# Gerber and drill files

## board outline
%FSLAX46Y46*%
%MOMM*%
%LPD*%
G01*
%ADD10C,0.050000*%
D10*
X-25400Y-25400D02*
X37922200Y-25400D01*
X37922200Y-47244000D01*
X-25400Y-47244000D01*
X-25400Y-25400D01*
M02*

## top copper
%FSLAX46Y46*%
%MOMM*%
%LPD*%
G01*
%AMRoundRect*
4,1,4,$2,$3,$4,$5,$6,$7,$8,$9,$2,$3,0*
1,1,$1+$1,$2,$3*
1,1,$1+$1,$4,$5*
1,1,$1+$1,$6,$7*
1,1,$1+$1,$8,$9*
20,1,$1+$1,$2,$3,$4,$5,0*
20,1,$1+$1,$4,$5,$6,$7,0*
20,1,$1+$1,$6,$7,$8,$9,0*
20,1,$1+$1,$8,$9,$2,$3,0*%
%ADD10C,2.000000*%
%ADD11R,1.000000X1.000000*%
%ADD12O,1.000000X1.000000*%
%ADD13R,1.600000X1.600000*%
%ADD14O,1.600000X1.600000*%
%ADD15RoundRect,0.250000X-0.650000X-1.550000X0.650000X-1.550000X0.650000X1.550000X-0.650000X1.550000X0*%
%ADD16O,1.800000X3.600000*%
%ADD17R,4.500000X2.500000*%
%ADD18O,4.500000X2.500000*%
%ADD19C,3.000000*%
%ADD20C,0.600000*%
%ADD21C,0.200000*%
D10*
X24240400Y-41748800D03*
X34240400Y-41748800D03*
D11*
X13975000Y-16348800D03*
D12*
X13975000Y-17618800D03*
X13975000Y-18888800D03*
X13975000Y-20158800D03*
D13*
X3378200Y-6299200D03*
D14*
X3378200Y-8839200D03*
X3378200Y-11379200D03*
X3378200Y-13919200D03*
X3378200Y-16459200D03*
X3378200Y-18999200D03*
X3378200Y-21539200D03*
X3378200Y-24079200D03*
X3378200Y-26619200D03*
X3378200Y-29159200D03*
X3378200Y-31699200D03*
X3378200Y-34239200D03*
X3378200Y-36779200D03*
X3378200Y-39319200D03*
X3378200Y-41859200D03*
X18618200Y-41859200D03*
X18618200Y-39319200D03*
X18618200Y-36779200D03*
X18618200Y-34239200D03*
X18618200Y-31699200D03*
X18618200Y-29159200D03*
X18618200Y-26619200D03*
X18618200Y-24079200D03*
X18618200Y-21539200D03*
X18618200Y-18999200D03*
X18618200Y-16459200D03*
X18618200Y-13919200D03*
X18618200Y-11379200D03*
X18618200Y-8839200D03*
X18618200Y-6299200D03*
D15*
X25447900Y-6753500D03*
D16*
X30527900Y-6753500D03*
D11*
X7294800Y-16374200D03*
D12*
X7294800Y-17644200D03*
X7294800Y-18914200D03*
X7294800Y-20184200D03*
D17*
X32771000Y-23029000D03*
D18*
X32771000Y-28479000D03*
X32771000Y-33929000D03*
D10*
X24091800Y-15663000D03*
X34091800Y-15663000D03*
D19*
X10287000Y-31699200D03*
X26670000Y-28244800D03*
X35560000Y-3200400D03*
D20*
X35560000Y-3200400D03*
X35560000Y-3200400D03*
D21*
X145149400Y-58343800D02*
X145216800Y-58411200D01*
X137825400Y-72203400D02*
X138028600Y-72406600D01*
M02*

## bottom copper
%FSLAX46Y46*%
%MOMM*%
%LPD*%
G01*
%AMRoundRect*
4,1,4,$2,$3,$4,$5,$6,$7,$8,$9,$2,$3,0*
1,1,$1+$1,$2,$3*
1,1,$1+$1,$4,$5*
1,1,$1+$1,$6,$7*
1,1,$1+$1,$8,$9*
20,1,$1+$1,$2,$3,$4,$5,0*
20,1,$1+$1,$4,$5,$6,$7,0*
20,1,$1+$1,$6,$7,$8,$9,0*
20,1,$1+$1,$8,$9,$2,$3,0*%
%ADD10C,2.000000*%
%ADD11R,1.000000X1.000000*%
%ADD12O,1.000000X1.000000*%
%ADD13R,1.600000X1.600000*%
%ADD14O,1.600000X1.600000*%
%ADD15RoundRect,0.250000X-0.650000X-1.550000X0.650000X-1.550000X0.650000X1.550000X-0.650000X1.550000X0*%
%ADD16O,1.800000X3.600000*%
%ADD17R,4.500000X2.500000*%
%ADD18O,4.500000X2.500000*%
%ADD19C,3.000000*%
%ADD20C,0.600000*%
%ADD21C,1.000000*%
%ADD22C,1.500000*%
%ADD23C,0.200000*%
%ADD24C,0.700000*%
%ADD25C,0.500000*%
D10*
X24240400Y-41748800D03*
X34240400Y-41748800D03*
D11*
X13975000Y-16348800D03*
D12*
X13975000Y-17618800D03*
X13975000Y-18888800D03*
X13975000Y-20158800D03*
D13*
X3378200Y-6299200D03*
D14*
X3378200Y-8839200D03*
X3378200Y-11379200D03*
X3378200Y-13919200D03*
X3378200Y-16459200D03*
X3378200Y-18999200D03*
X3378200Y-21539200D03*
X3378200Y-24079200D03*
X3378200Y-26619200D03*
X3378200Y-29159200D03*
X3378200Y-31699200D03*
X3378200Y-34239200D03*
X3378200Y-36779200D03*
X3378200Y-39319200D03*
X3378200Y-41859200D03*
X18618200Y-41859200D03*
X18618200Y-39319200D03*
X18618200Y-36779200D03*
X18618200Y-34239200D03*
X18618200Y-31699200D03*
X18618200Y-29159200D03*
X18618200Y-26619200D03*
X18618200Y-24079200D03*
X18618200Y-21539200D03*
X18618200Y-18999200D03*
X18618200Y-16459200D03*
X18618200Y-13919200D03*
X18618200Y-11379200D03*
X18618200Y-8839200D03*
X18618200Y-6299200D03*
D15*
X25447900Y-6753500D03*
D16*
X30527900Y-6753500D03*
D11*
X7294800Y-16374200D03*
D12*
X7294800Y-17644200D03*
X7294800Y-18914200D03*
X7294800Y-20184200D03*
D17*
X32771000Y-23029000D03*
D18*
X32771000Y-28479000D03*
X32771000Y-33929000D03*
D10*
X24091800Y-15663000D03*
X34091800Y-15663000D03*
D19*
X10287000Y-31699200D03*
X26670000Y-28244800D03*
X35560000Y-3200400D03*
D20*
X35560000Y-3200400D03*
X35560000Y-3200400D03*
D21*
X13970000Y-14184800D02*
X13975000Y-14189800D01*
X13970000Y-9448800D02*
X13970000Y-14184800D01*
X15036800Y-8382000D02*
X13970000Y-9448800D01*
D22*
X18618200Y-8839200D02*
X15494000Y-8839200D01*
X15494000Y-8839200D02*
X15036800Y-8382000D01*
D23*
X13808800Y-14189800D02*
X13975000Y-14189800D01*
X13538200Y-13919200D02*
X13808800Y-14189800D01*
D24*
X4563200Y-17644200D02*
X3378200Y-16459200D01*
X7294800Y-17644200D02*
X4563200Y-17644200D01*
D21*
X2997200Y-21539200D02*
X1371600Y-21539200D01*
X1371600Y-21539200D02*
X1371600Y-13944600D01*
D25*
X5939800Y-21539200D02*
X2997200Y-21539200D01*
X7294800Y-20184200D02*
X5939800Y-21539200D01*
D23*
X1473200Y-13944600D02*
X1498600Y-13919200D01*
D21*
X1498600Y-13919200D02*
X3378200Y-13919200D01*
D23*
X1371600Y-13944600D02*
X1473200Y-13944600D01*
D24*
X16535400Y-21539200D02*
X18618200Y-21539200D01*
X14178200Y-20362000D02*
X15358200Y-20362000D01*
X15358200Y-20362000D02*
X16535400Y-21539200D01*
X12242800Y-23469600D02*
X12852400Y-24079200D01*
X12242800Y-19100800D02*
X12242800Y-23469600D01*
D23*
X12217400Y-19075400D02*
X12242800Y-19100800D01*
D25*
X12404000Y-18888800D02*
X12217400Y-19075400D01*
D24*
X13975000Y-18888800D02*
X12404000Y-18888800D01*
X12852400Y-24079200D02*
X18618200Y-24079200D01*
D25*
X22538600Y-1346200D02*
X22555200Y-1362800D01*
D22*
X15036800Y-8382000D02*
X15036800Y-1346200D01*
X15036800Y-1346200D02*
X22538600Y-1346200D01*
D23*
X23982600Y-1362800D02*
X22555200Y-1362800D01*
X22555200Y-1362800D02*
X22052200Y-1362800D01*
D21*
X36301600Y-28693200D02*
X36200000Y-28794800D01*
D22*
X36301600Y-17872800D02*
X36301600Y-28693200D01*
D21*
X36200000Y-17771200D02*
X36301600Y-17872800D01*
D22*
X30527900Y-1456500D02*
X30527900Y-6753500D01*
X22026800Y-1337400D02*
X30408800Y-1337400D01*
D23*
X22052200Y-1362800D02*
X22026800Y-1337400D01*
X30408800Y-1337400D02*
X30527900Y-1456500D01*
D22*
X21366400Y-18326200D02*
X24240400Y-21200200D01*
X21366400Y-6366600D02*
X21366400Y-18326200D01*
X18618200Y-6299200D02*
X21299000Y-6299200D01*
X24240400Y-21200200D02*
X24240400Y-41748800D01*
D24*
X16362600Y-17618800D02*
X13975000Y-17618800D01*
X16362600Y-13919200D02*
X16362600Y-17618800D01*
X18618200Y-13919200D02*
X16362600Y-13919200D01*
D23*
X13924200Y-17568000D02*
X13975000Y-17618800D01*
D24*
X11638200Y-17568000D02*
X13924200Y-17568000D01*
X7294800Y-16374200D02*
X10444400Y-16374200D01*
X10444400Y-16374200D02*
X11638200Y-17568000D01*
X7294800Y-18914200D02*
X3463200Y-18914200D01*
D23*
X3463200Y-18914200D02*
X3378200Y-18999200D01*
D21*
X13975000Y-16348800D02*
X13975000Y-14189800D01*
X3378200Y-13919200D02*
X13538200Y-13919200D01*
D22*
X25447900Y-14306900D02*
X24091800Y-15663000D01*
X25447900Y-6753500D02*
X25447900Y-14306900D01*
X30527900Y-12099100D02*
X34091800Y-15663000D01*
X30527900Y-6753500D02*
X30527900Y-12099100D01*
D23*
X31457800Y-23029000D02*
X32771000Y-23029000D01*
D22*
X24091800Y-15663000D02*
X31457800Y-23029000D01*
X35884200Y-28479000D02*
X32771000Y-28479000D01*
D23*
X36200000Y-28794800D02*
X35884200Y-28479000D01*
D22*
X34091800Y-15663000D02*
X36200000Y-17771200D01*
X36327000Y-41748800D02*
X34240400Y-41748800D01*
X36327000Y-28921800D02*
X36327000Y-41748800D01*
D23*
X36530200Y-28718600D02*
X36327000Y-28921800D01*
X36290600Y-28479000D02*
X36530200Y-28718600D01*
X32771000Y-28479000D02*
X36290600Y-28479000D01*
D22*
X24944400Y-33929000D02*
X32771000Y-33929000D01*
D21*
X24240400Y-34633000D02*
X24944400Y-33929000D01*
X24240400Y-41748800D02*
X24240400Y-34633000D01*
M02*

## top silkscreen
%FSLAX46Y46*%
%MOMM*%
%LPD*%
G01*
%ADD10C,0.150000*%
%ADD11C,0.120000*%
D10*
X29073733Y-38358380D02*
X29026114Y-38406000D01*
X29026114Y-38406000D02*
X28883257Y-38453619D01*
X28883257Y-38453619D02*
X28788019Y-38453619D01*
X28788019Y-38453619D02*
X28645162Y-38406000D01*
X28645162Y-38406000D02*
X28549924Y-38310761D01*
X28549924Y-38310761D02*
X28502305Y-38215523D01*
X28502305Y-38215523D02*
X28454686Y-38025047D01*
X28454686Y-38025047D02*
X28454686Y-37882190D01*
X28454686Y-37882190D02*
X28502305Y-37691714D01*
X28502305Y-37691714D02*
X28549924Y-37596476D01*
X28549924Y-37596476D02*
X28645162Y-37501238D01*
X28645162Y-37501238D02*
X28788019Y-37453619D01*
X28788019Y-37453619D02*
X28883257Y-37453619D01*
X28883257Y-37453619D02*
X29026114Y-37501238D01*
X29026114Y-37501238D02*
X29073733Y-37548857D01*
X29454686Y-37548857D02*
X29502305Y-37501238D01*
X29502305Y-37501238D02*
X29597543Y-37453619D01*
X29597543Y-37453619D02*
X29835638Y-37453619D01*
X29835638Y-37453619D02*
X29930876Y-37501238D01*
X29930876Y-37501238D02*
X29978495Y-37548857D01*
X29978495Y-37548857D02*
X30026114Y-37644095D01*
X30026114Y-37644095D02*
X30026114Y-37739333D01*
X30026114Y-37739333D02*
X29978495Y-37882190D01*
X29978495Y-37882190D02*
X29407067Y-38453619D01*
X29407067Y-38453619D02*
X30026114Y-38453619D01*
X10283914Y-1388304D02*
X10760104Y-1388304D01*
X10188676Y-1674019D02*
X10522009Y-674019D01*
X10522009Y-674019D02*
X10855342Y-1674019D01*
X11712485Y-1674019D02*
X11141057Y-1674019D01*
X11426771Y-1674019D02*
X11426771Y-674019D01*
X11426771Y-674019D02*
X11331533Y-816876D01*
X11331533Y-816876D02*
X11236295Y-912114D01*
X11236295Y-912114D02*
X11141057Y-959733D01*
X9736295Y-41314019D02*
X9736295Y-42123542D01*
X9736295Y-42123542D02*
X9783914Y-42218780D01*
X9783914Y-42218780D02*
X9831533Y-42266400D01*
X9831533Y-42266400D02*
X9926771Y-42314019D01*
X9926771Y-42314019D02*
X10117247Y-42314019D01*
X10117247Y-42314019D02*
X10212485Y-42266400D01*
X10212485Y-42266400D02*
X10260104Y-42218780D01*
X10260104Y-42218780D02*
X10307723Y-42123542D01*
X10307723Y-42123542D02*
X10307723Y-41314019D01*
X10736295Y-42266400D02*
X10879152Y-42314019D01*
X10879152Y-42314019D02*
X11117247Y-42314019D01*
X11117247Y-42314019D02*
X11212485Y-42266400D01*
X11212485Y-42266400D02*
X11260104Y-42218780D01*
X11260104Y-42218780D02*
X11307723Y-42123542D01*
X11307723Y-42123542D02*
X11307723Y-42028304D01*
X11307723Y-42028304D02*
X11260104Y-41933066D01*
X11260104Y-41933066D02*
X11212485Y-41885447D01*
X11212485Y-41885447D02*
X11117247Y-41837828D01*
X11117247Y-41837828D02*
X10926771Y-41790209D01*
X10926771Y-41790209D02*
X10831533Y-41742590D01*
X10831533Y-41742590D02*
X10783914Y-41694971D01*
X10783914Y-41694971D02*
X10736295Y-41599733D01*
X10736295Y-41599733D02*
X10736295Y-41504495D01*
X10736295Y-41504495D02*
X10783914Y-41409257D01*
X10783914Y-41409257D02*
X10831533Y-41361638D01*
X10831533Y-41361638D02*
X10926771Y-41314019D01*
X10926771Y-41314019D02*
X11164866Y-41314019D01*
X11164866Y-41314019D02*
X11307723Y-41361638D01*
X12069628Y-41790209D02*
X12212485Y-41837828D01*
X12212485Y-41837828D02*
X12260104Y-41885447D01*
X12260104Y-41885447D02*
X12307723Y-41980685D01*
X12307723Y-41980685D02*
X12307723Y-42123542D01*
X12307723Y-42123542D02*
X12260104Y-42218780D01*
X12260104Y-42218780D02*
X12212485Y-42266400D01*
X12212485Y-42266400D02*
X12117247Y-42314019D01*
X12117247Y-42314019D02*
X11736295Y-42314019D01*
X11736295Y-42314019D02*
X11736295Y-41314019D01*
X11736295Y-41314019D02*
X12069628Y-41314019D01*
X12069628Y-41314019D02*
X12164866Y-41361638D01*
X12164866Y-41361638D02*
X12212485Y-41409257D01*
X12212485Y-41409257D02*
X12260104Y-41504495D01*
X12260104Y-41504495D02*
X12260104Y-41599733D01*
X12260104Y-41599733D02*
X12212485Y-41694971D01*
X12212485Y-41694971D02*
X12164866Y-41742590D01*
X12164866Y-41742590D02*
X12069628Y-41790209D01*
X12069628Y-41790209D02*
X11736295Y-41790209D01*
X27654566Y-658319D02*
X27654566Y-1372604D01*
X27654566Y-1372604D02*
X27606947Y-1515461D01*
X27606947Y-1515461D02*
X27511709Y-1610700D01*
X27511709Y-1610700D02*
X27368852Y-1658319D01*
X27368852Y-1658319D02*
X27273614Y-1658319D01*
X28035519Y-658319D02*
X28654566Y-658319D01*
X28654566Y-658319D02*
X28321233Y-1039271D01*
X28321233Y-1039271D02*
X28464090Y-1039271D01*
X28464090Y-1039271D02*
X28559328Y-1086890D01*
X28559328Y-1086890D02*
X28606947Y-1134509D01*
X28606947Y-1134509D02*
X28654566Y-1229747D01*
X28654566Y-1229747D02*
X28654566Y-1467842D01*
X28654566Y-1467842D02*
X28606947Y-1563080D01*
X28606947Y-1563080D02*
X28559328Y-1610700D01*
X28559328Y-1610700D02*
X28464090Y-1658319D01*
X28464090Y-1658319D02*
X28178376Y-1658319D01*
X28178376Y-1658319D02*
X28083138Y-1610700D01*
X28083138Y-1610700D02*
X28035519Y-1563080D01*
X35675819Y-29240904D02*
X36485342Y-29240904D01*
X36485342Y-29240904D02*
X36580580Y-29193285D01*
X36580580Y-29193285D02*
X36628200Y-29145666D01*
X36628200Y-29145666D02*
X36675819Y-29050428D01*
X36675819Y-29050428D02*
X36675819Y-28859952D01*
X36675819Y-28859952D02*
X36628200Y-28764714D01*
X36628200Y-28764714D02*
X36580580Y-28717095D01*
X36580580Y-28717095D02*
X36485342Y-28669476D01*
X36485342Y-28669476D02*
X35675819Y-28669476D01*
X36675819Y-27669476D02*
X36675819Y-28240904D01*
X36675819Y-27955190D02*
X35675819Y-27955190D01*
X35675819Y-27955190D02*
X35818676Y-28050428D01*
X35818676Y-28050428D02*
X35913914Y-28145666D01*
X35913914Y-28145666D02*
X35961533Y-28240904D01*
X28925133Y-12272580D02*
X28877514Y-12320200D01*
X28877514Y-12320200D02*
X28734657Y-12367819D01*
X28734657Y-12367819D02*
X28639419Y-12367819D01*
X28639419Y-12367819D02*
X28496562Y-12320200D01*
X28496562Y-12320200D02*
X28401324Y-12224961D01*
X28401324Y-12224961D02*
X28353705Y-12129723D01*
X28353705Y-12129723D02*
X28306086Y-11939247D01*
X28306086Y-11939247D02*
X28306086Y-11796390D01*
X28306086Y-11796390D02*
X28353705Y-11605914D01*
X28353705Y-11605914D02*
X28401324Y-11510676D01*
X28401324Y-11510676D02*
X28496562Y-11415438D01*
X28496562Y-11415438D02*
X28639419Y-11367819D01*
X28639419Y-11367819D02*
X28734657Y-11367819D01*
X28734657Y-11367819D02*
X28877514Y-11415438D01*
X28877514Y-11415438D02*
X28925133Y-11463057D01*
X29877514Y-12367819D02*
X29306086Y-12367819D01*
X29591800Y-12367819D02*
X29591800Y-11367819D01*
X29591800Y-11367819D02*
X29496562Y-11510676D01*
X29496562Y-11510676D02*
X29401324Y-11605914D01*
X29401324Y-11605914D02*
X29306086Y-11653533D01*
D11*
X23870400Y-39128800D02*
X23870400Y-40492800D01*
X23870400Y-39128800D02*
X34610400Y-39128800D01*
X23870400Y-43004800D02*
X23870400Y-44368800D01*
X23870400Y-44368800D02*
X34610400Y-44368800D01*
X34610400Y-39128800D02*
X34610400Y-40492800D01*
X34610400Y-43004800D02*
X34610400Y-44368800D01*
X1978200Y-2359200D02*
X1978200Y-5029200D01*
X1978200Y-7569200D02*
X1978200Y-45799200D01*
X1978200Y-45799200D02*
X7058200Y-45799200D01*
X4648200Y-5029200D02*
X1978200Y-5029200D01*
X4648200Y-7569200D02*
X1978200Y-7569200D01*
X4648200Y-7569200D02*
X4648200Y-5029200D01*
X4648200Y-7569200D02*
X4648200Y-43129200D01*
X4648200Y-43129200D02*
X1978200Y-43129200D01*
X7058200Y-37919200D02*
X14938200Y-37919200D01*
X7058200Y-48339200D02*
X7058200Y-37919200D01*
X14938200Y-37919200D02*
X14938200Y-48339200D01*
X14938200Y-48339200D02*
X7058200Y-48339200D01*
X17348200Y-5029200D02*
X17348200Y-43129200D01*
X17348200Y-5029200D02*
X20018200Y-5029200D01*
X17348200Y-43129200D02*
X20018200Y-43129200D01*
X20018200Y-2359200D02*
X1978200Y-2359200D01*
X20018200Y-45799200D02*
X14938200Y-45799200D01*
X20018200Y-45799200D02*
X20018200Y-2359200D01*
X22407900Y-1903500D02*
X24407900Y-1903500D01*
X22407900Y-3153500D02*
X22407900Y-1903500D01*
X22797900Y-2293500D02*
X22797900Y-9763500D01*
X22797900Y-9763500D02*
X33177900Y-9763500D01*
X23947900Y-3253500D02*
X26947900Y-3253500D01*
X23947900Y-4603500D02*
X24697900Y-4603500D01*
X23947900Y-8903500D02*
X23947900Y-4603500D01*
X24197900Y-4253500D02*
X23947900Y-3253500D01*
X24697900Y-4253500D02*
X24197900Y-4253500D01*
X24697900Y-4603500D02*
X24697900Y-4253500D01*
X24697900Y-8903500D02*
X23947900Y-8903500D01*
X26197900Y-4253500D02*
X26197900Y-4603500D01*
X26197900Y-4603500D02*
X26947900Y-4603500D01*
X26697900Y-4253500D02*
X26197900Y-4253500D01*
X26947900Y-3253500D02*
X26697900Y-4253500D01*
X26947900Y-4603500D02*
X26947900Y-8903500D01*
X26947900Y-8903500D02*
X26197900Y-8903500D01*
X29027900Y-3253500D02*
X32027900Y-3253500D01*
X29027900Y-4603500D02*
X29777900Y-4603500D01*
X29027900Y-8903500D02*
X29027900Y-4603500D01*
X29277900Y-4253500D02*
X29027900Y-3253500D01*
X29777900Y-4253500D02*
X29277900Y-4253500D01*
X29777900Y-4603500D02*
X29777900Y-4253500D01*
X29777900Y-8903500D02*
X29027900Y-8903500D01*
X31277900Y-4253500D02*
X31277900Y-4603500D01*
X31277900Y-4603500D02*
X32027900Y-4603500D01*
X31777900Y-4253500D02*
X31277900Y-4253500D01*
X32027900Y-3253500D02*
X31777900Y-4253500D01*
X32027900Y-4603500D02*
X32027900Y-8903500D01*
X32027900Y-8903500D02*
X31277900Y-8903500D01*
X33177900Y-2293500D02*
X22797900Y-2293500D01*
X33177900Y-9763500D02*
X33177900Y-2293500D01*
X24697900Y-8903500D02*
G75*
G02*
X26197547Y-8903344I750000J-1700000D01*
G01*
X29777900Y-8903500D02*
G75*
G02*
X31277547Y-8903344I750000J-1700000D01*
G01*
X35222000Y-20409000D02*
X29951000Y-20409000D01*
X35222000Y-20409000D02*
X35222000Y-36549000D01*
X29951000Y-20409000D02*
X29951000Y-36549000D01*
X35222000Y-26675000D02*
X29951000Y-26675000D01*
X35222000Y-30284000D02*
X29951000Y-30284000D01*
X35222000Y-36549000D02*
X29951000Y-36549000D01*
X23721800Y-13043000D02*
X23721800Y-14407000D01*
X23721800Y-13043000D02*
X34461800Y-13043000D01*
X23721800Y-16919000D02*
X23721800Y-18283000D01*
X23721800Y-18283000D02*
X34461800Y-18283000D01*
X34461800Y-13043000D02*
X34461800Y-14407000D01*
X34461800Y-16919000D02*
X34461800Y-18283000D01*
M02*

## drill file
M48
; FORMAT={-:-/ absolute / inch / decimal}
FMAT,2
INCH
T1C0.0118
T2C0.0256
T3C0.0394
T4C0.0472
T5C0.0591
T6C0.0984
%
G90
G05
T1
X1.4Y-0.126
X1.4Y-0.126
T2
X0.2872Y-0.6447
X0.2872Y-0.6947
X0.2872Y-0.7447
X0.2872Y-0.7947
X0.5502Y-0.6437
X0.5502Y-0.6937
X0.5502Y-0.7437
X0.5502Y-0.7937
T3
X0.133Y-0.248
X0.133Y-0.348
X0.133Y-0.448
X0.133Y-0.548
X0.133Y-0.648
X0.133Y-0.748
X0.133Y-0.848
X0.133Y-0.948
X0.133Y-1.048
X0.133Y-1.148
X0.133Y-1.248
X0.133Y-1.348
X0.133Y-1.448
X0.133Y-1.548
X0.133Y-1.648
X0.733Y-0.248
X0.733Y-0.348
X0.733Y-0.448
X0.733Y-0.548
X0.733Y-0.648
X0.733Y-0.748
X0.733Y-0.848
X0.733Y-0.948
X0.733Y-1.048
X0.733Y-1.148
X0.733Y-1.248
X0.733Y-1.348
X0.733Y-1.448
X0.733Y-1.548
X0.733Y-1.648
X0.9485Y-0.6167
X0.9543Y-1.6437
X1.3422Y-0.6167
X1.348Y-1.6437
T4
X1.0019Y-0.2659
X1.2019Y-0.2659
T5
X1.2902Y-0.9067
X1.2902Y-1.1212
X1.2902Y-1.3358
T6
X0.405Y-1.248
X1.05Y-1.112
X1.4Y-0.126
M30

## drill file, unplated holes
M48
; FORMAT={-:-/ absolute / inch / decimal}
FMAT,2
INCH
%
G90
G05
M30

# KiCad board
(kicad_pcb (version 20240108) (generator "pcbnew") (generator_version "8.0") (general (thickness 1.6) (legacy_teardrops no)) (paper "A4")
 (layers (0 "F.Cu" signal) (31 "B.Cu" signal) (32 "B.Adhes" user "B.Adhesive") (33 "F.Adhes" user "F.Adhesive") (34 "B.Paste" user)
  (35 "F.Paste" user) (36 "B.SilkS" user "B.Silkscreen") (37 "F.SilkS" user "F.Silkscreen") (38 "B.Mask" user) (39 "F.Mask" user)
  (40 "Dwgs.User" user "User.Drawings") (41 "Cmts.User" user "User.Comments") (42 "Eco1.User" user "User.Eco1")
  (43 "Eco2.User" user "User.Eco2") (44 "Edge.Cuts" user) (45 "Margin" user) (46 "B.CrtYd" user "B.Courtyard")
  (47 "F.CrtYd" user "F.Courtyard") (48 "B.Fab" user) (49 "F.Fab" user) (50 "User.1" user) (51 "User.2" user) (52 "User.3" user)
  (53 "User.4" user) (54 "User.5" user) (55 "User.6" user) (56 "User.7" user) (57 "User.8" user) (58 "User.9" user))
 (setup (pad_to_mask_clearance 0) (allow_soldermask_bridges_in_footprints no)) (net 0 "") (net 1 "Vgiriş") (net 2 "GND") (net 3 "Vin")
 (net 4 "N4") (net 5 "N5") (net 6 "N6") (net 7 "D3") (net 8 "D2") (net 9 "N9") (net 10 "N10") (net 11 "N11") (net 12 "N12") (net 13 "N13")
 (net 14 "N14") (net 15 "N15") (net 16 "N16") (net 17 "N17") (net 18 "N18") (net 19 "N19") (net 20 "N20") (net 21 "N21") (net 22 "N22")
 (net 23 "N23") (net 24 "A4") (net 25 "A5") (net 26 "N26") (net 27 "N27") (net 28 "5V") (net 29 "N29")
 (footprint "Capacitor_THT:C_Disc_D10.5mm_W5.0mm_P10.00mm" (layer "F.Cu") (at 24.0918 15.663)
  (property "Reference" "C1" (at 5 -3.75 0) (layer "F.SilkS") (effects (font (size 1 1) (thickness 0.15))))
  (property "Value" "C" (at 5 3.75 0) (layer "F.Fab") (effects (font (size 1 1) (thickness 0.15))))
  (fp_line (start -0.37 -2.62) (end -0.37 -1.256) (stroke (width 0.12) (type solid)) (layer "F.SilkS"))
  (fp_line (start -0.37 -2.62) (end 10.37 -2.62) (stroke (width 0.12) (type solid)) (layer "F.SilkS"))
  (fp_line (start -0.37 1.256) (end -0.37 2.62) (stroke (width 0.12) (type solid)) (layer "F.SilkS"))
  (fp_line (start -0.37 2.62) (end 10.37 2.62) (stroke (width 0.12) (type solid)) (layer "F.SilkS"))
  (fp_line (start 10.37 -2.62) (end 10.37 -1.256) (stroke (width 0.12) (type solid)) (layer "F.SilkS"))
  (fp_line (start 10.37 1.256) (end 10.37 2.62) (stroke (width 0.12) (type solid)) (layer "F.SilkS"))
  (pad "1" thru_hole circle (at 0 0) (size 2 2) (drill 1) (layers "*.Cu" "*.Mask") (remove_unused_layers no) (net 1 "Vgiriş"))
  (pad "2" thru_hole circle (at 10 0) (size 2 2) (drill 1) (layers "*.Cu" "*.Mask") (remove_unused_layers no) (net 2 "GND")))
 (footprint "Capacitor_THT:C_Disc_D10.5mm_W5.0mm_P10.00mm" (layer "F.Cu") (at 24.2404 41.7488)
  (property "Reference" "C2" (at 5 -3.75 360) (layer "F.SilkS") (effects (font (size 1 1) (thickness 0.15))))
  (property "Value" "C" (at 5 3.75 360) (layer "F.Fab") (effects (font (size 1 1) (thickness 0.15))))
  (fp_line (start -0.37 -2.62) (end -0.37 -1.256) (stroke (width 0.12) (type solid)) (layer "F.SilkS"))
  (fp_line (start -0.37 -2.62) (end 10.37 -2.62) (stroke (width 0.12) (type solid)) (layer "F.SilkS"))
  (fp_line (start -0.37 1.256) (end -0.37 2.62) (stroke (width 0.12) (type solid)) (layer "F.SilkS"))
  (fp_line (start -0.37 2.62) (end 10.37 2.62) (stroke (width 0.12) (type solid)) (layer "F.SilkS"))
  (fp_line (start 10.37 -2.62) (end 10.37 -1.256) (stroke (width 0.12) (type solid)) (layer "F.SilkS"))
  (fp_line (start 10.37 1.256) (end 10.37 2.62) (stroke (width 0.12) (type solid)) (layer "F.SilkS"))
  (pad "1" thru_hole circle (at 0 0) (size 2 2) (drill 1) (layers "*.Cu" "*.Mask") (remove_unused_layers no) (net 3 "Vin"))
  (pad "2" thru_hole circle (at 10 0) (size 2 2) (drill 1) (layers "*.Cu" "*.Mask") (remove_unused_layers no) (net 2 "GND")))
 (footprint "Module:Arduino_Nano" (layer "F.Cu") (at 3.3782 6.2992)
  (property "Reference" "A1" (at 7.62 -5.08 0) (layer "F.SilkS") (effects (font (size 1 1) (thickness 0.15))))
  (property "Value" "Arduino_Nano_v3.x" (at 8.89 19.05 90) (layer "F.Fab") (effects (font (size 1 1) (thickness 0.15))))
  (fp_line (start -1.4 -3.94) (end -1.4 -1.27) (stroke (width 0.12) (type solid)) (layer "F.SilkS"))
  (fp_line (start -1.4 1.27) (end -1.4 39.5) (stroke (width 0.12) (type solid)) (layer "F.SilkS"))
  (fp_line (start -1.4 39.5) (end 3.68 39.5) (stroke (width 0.12) (type solid)) (layer "F.SilkS"))
  (fp_line (start 1.27 -1.27) (end -1.4 -1.27) (stroke (width 0.12) (type solid)) (layer "F.SilkS"))
  (fp_line (start 1.27 1.27) (end -1.4 1.27) (stroke (width 0.12) (type solid)) (layer "F.SilkS"))
  (fp_line (start 1.27 1.27) (end 1.27 -1.27) (stroke (width 0.12) (type solid)) (layer "F.SilkS"))
  (fp_line (start 1.27 1.27) (end 1.27 36.83) (stroke (width 0.12) (type solid)) (layer "F.SilkS"))
  (fp_line (start 1.27 36.83) (end -1.4 36.83) (stroke (width 0.12) (type solid)) (layer "F.SilkS"))
  (fp_line (start 3.68 31.62) (end 11.56 31.62) (stroke (width 0.12) (type solid)) (layer "F.SilkS"))
  (fp_line (start 3.68 42.04) (end 3.68 31.62) (stroke (width 0.12) (type solid)) (layer "F.SilkS"))
  (fp_line (start 11.56 31.62) (end 11.56 42.04) (stroke (width 0.12) (type solid)) (layer "F.SilkS"))
  (fp_line (start 11.56 42.04) (end 3.68 42.04) (stroke (width 0.12) (type solid)) (layer "F.SilkS"))
  (fp_line (start 13.97 -1.27) (end 13.97 36.83) (stroke (width 0.12) (type solid)) (layer "F.SilkS"))
  (fp_line (start 13.97 -1.27) (end 16.64 -1.27) (stroke (width 0.12) (type solid)) (layer "F.SilkS"))
  (fp_line (start 13.97 36.83) (end 16.64 36.83) (stroke (width 0.12) (type solid)) (layer "F.SilkS"))
  (fp_line (start 16.64 -3.94) (end -1.4 -3.94) (stroke (width 0.12) (type solid)) (layer "F.SilkS"))
  (fp_line (start 16.64 39.5) (end 11.56 39.5) (stroke (width 0.12) (type solid)) (layer "F.SilkS"))
  (fp_line (start 16.64 39.5) (end 16.64 -3.94) (stroke (width 0.12) (type solid)) (layer "F.SilkS"))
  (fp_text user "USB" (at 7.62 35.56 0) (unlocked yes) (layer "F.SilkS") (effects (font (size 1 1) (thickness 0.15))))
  (pad "1" thru_hole rect (at 0 0) (size 1.6 1.6) (drill 1) (layers "*.Cu" "*.Mask") (remove_unused_layers no) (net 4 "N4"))
  (pad "2" thru_hole oval (at 0 2.54) (size 1.6 1.6) (drill 1) (layers "*.Cu" "*.Mask") (remove_unused_layers no) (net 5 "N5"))
  (pad "3" thru_hole oval (at 0 5.08) (size 1.6 1.6) (drill 1) (layers "*.Cu" "*.Mask") (remove_unused_layers no) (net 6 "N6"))
  (pad "4" thru_hole oval (at 0 7.62) (size 1.6 1.6) (drill 1) (layers "*.Cu" "*.Mask") (remove_unused_layers no) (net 2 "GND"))
  (pad "5" thru_hole oval (at 0 10.16) (size 1.6 1.6) (drill 1) (layers "*.Cu" "*.Mask") (remove_unused_layers no) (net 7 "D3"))
  (pad "6" thru_hole oval (at 0 12.7) (size 1.6 1.6) (drill 1) (layers "*.Cu" "*.Mask") (remove_unused_layers no) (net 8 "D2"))
  (pad "7" thru_hole oval (at 0 15.24) (size 1.6 1.6) (drill 1) (layers "*.Cu" "*.Mask") (remove_unused_layers no) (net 2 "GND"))
  (pad "8" thru_hole oval (at 0 17.78) (size 1.6 1.6) (drill 1) (layers "*.Cu" "*.Mask") (remove_unused_layers no) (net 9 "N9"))
  (pad "9" thru_hole oval (at 0 20.32) (size 1.6 1.6) (drill 1) (layers "*.Cu" "*.Mask") (remove_unused_layers no) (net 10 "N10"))
  (pad "10" thru_hole oval (at 0 22.86) (size 1.6 1.6) (drill 1) (layers "*.Cu" "*.Mask") (remove_unused_layers no) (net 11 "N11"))
  (pad "11" thru_hole oval (at 0 25.4) (size 1.6 1.6) (drill 1) (layers "*.Cu" "*.Mask") (remove_unused_layers no) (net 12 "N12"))
  (pad "12" thru_hole oval (at 0 27.94) (size 1.6 1.6) (drill 1) (layers "*.Cu" "*.Mask") (remove_unused_layers no) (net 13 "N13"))
  (pad "13" thru_hole oval (at 0 30.48) (size 1.6 1.6) (drill 1) (layers "*.Cu" "*.Mask") (remove_unused_layers no) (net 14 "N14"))
  (pad "14" thru_hole oval (at 0 33.02) (size 1.6 1.6) (drill 1) (layers "*.Cu" "*.Mask") (remove_unused_layers no) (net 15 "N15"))
  (pad "15" thru_hole oval (at 0 35.56) (size 1.6 1.6) (drill 1) (layers "*.Cu" "*.Mask") (remove_unused_layers no) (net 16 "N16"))
  (pad "16" thru_hole oval (at 15.24 35.56) (size 1.6 1.6) (drill 1) (layers "*.Cu" "*.Mask") (remove_unused_layers no) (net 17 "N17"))
  (pad "17" thru_hole oval (at 15.24 33.02) (size 1.6 1.6) (drill 1) (layers "*.Cu" "*.Mask") (remove_unused_layers no) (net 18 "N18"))
  (pad "18" thru_hole oval (at 15.24 30.48) (size 1.6 1.6) (drill 1) (layers "*.Cu" "*.Mask") (remove_unused_layers no) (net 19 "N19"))
  (pad "19" thru_hole oval (at 15.24 27.94) (size 1.6 1.6) (drill 1) (layers "*.Cu" "*.Mask") (remove_unused_layers no) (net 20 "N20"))
  (pad "20" thru_hole oval (at 15.24 25.4) (size 1.6 1.6) (drill 1) (layers "*.Cu" "*.Mask") (remove_unused_layers no) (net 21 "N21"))
  (pad "21" thru_hole oval (at 15.24 22.86) (size 1.6 1.6) (drill 1) (layers "*.Cu" "*.Mask") (remove_unused_layers no) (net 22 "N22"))
  (pad "22" thru_hole oval (at 15.24 20.32) (size 1.6 1.6) (drill 1) (layers "*.Cu" "*.Mask") (remove_unused_layers no) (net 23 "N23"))
  (pad "23" thru_hole oval (at 15.24 17.78) (size 1.6 1.6) (drill 1) (layers "*.Cu" "*.Mask") (remove_unused_layers no) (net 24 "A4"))
  (pad "24" thru_hole oval (at 15.24 15.24) (size 1.6 1.6) (drill 1) (layers "*.Cu" "*.Mask") (remove_unused_layers no) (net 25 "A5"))
  (pad "25" thru_hole oval (at 15.24 12.7) (size 1.6 1.6) (drill 1) (layers "*.Cu" "*.Mask") (remove_unused_layers no) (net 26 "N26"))
  (pad "26" thru_hole oval (at 15.24 10.16) (size 1.6 1.6) (drill 1) (layers "*.Cu" "*.Mask") (remove_unused_layers no) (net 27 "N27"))
  (pad "27" thru_hole oval (at 15.24 7.62) (size 1.6 1.6) (drill 1) (layers "*.Cu" "*.Mask") (remove_unused_layers no) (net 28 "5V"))
  (pad "28" thru_hole oval (at 15.24 5.08) (size 1.6 1.6) (drill 1) (layers "*.Cu" "*.Mask") (remove_unused_layers no) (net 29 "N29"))
  (pad "29" thru_hole oval (at 15.24 2.54) (size 1.6 1.6) (drill 1) (layers "*.Cu" "*.Mask") (remove_unused_layers no) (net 2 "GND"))
  (pad "30" thru_hole oval (at 15.24 0) (size 1.6 1.6) (drill 1) (layers "*.Cu" "*.Mask") (remove_unused_layers no) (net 3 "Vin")))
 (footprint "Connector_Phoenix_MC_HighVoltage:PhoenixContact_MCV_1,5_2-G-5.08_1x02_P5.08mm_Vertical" (layer "F.Cu") (at 25.4479 6.7535)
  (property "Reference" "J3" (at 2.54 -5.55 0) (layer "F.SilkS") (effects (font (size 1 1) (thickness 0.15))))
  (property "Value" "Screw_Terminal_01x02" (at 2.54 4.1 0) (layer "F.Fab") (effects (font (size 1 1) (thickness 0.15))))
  (fp_line (start -3.04 -4.85) (end -1.04 -4.85) (stroke (width 0.12) (type solid)) (layer "F.SilkS"))
  (fp_line (start -3.04 -3.6) (end -3.04 -4.85) (stroke (width 0.12) (type solid)) (layer "F.SilkS"))
  (fp_line (start -2.65 -4.46) (end -2.65 3.01) (stroke (width 0.12) (type solid)) (layer "F.SilkS"))
  (fp_line (start -2.65 3.01) (end 7.73 3.01) (stroke (width 0.12) (type solid)) (layer "F.SilkS"))
  (fp_line (start -1.5 -3.5) (end 1.5 -3.5) (stroke (width 0.12) (type solid)) (layer "F.SilkS"))
  (fp_line (start -1.5 -2.15) (end -0.75 -2.15) (stroke (width 0.12) (type solid)) (layer "F.SilkS"))
  (fp_line (start -1.5 2.15) (end -1.5 -2.15) (stroke (width 0.12) (type solid)) (layer "F.SilkS"))
  (fp_line (start -1.25 -2.5) (end -1.5 -3.5) (stroke (width 0.12) (type solid)) (layer "F.SilkS"))
  (fp_line (start -0.75 -2.5) (end -1.25 -2.5) (stroke (width 0.12) (type solid)) (layer "F.SilkS"))
  (fp_line (start -0.75 -2.15) (end -0.75 -2.5) (stroke (width 0.12) (type solid)) (layer "F.SilkS"))
  (fp_line (start -0.75 2.15) (end -1.5 2.15) (stroke (width 0.12) (type solid)) (layer "F.SilkS"))
  (fp_line (start 0.75 -2.5) (end 0.75 -2.15) (stroke (width 0.12) (type solid)) (layer "F.SilkS"))
  (fp_line (start 0.75 -2.15) (end 1.5 -2.15) (stroke (width 0.12) (type solid)) (layer "F.SilkS"))
  (fp_line (start 1.25 -2.5) (end 0.75 -2.5) (stroke (width 0.12) (type solid)) (layer "F.SilkS"))
  (fp_line (start 1.5 -3.5) (end 1.25 -2.5) (stroke (width 0.12) (type solid)) (layer "F.SilkS"))
  (fp_line (start 1.5 -2.15) (end 1.5 2.15) (stroke (width 0.12) (type solid)) (layer "F.SilkS"))
  (fp_line (start 1.5 2.15) (end 0.75 2.15) (stroke (width 0.12) (type solid)) (layer "F.SilkS"))
  (fp_line (start 3.58 -3.5) (end 6.58 -3.5) (stroke (width 0.12) (type solid)) (layer "F.SilkS"))
  (fp_line (start 3.58 -2.15) (end 4.33 -2.15) (stroke (width 0.12) (type solid)) (layer "F.SilkS"))
  (fp_line (start 3.58 2.15) (end 3.58 -2.15) (stroke (width 0.12) (type solid)) (layer "F.SilkS"))
  (fp_line (start 3.83 -2.5) (end 3.58 -3.5) (stroke (width 0.12) (type solid)) (layer "F.SilkS"))
  (fp_line (start 4.33 -2.5) (end 3.83 -2.5) (stroke (width 0.12) (type solid)) (layer "F.SilkS"))
  (fp_line (start 4.33 -2.15) (end 4.33 -2.5) (stroke (width 0.12) (type solid)) (layer "F.SilkS"))
  (fp_line (start 4.33 2.15) (end 3.58 2.15) (stroke (width 0.12) (type solid)) (layer "F.SilkS"))
  (fp_line (start 5.83 -2.5) (end 5.83 -2.15) (stroke (width 0.12) (type solid)) (layer "F.SilkS"))
  (fp_line (start 5.83 -2.15) (end 6.58 -2.15) (stroke (width 0.12) (type solid)) (layer "F.SilkS"))
  (fp_line (start 6.33 -2.5) (end 5.83 -2.5) (stroke (width 0.12) (type solid)) (layer "F.SilkS"))
  (fp_line (start 6.58 -3.5) (end 6.33 -2.5) (stroke (width 0.12) (type solid)) (layer "F.SilkS"))
  (fp_line (start 6.58 -2.15) (end 6.58 2.15) (stroke (width 0.12) (type solid)) (layer "F.SilkS"))
  (fp_line (start 6.58 2.15) (end 5.83 2.15) (stroke (width 0.12) (type solid)) (layer "F.SilkS"))
  (fp_line (start 7.73 -4.46) (end -2.65 -4.46) (stroke (width 0.12) (type solid)) (layer "F.SilkS"))
  (fp_line (start 7.73 3.01) (end 7.73 -4.46) (stroke (width 0.12) (type solid)) (layer "F.SilkS"))
  (fp_arc (start -0.75 2.15) (mid -0.000193 1.99191) (end 0.749647 2.149844) (stroke (width 0.12) (type solid)) (layer "F.SilkS"))
  (fp_arc (start 4.33 2.15) (mid 5.079807 1.99191) (end 5.829647 2.149844) (stroke (width 0.12) (type solid)) (layer "F.SilkS"))
  (pad "1" thru_hole roundrect (at 0 0) (size 1.8 3.6) (drill 1.2) (layers "*.Cu" "*.Mask") (remove_unused_layers no)
   (roundrect_rratio 0.138889) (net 1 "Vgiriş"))
  (pad "2" thru_hole oval (at 5.08 0) (size 1.8 3.6) (drill 1.2) (layers "*.Cu" "*.Mask") (remove_unused_layers no) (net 2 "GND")))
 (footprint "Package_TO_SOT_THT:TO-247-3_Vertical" (layer "F.Cu") (at 32.771 23.029 -90)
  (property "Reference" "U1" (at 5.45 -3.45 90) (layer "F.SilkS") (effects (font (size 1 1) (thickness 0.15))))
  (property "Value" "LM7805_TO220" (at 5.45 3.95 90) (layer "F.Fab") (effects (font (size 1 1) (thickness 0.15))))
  (fp_line (start -2.62 2.82) (end 13.52 2.82) (stroke (width 0.12) (type solid)) (layer "F.SilkS"))
  (fp_line (start -2.62 -2.451) (end -2.62 2.82) (stroke (width 0.12) (type solid)) (layer "F.SilkS"))
  (fp_line (start -2.62 -2.451) (end 13.52 -2.451) (stroke (width 0.12) (type solid)) (layer "F.SilkS"))
  (fp_line (start 3.646 -2.451) (end 3.646 2.82) (stroke (width 0.12) (type solid)) (layer "F.SilkS"))
  (fp_line (start 7.255 -2.451) (end 7.255 2.82) (stroke (width 0.12) (type solid)) (layer "F.SilkS"))
  (fp_line (start 13.52 -2.451) (end 13.52 2.82) (stroke (width 0.12) (type solid)) (layer "F.SilkS"))
  (pad "1" thru_hole rect (at 0 0 270) (size 2.5 4.5) (drill 1.5) (layers "*.Cu" "*.Mask") (remove_unused_layers no) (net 1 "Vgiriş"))
  (pad "2" thru_hole oval (at 5.45 0 270) (size 2.5 4.5) (drill 1.5) (layers "*.Cu" "*.Mask") (remove_unused_layers no) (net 2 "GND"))
  (pad "3" thru_hole oval (at 10.9 0 270) (size 2.5 4.5) (drill 1.5) (layers "*.Cu" "*.Mask") (remove_unused_layers no) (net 3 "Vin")))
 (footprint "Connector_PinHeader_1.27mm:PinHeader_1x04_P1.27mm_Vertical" (layer "B.Cu") (at 13.975 16.3488 180)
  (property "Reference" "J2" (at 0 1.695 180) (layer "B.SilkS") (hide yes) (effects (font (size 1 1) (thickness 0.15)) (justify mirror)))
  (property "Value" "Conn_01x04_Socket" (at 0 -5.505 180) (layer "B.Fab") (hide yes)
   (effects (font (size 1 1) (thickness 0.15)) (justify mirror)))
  (pad "1" thru_hole rect (at 0 0 180) (size 1 1) (drill 0.65) (layers "*.Cu" "*.Mask") (remove_unused_layers no) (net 2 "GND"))
  (pad "2" thru_hole oval (at 0 -1.27 180) (size 1 1) (drill 0.65) (layers "*.Cu" "*.Mask") (remove_unused_layers no) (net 28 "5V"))
  (pad "3" thru_hole oval (at 0 -2.54 180) (size 1 1) (drill 0.65) (layers "*.Cu" "*.Mask") (remove_unused_layers no) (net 24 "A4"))
  (pad "4" thru_hole oval (at 0 -3.81 180) (size 1 1) (drill 0.65) (layers "*.Cu" "*.Mask") (remove_unused_layers no) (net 25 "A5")))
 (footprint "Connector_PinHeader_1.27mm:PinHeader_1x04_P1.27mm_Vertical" (layer "B.Cu") (at 7.2948 16.3742 180)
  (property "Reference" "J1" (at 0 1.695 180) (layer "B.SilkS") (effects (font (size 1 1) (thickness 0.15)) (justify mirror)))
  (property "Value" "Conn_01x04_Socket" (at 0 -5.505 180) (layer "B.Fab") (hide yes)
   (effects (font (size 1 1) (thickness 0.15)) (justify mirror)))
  (pad "1" thru_hole rect (at 0 0 180) (size 1 1) (drill 0.65) (layers "*.Cu" "*.Mask") (remove_unused_layers no) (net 28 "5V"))
  (pad "2" thru_hole oval (at 0 -1.27 180) (size 1 1) (drill 0.65) (layers "*.Cu" "*.Mask") (remove_unused_layers no) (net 7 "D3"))
  (pad "3" thru_hole oval (at 0 -2.54 180) (size 1 1) (drill 0.65) (layers "*.Cu" "*.Mask") (remove_unused_layers no) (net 8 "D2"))
  (pad "4" thru_hole oval (at 0 -3.81 180) (size 1 1) (drill 0.65) (layers "*.Cu" "*.Mask") (remove_unused_layers no) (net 2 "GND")))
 (gr_rect (start -0.0254 0.0254) (end 37.9222 47.244) (stroke (width 0.05) (type default)) (fill none) (layer "Edge.Cuts"))
 (via (at 10.287 31.6992) (size 3) (drill 2.5) (layers "F.Cu" "B.Cu") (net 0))
 (via (at 35.56 3.2004) (size 0.6) (drill 0.3) (layers "F.Cu" "B.Cu") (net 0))
 (via (at 35.56 3.2004) (size 0.6) (drill 0.3) (layers "F.Cu" "B.Cu") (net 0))
 (via (at 26.67 28.2448) (size 3) (drill 2.5) (layers "F.Cu" "B.Cu") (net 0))
 (via (at 35.56 3.2004) (size 3) (drill 2.5) (layers "F.Cu" "B.Cu") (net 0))
 (segment (start 4.5632 17.6442) (end 3.3782 16.4592) (width 0.7) (layer "B.Cu") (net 7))
 (segment (start 7.2948 17.6442) (end 4.5632 17.6442) (width 0.7) (layer "B.Cu") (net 7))
 (segment (start 1.4986 13.9192) (end 3.3782 13.9192) (width 1) (layer "B.Cu") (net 2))
 (segment (start 5.9398 21.5392) (end 2.9972 21.5392) (width 0.5) (layer "B.Cu") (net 2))
 (segment (start 15.0368 8.382) (end 15.0368 1.3462) (width 1.5) (layer "B.Cu") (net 2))
 (segment (start 23.9826 1.3628) (end 22.5552 1.3628) (width 0.2) (layer "B.Cu") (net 2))
 (segment (start 13.5382 13.9192) (end 13.8088 14.1898) (width 0.2) (layer "B.Cu") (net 2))
 (segment (start 30.5279 1.4565) (end 30.5279 6.7535) (width 1.5) (layer "B.Cu") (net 2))
 (segment (start 7.2948 20.1842) (end 5.9398 21.5392) (width 0.5) (layer "B.Cu") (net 2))
 (segment (start 18.6182 8.8392) (end 15.494 8.8392) (width 1.5) (layer "B.Cu") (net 2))
 (segment (start 36.2 17.7712) (end 36.3016 17.8728) (width 1) (layer "B.Cu") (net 2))
 (segment (start 30.5279 6.7535) (end 30.5279 12.0991) (width 1.5) (layer "B.Cu") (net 2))
 (segment (start 13.97 9.4488) (end 13.97 14.1848) (width 1) (layer "B.Cu") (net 2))
 (segment (start 15.0368 8.382) (end 13.97 9.4488) (width 1) (layer "B.Cu") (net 2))
 (segment (start 1.4732 13.9446) (end 1.4986 13.9192) (width 0.2) (layer "B.Cu") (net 2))
 (segment (start 36.2 28.7948) (end 35.8842 28.479) (width 0.2) (layer "B.Cu") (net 2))
 (segment (start 3.3782 13.9192) (end 13.5382 13.9192) (width 1) (layer "B.Cu") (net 2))
 (segment (start 34.0918 15.663) (end 36.2 17.7712) (width 1.5) (layer "B.Cu") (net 2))
 (segment (start 22.5552 1.3628) (end 22.0522 1.3628) (width 0.2) (layer "B.Cu") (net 2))
 (segment (start 35.8842 28.479) (end 32.771 28.479) (width 1.5) (layer "B.Cu") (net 2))
 (segment (start 22.0268 1.3374) (end 30.4088 1.3374) (width 1.5) (layer "B.Cu") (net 2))
 (segment (start 36.3016 28.6932) (end 36.2 28.7948) (width 1) (layer "B.Cu") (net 2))
 (segment (start 13.8088 14.1898) (end 13.975 14.1898) (width 0.2) (layer "B.Cu") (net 2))
 (segment (start 36.2906 28.479) (end 36.5302 28.7186) (width 0.2) (layer "B.Cu") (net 2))
 (segment (start 1.3716 13.9446) (end 1.4732 13.9446) (width 0.2) (layer "B.Cu") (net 2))
 (segment (start 1.3716 21.5392) (end 1.3716 13.9446) (width 1) (layer "B.Cu") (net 2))
 (segment (start 32.771 28.479) (end 36.2906 28.479) (width 0.2) (layer "B.Cu") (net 2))
 (segment (start 36.327 41.7488) (end 34.2404 41.7488) (width 1.5) (layer "B.Cu") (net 2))
 (segment (start 36.327 28.9218) (end 36.327 41.7488) (width 1.5) (layer "B.Cu") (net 2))
 (segment (start 13.97 14.1848) (end 13.975 14.1898) (width 1) (layer "B.Cu") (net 2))
 (segment (start 15.0368 1.3462) (end 22.5386 1.3462) (width 1.5) (layer "B.Cu") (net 2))
 (segment (start 15.494 8.8392) (end 15.0368 8.382) (width 1.5) (layer "B.Cu") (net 2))
 (segment (start 36.5302 28.7186) (end 36.327 28.9218) (width 0.2) (layer "B.Cu") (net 2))
 (segment (start 22.0522 1.3628) (end 22.0268 1.3374) (width 0.2) (layer "B.Cu") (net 2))
 (segment (start 36.3016 17.8728) (end 36.3016 28.6932) (width 1.5) (layer "B.Cu") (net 2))
 (segment (start 30.4088 1.3374) (end 30.5279 1.4565) (width 0.2) (layer "B.Cu") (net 2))
 (segment (start 30.5279 12.0991) (end 34.0918 15.663) (width 1.5) (layer "B.Cu") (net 2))
 (segment (start 2.9972 21.5392) (end 1.3716 21.5392) (width 1) (layer "B.Cu") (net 2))
 (segment (start 22.5386 1.3462) (end 22.5552 1.3628) (width 0.5) (layer "B.Cu") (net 2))
 (segment (start 13.975 16.3488) (end 13.975 14.1898) (width 1) (layer "B.Cu") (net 2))
 (segment (start 10.4444 16.3742) (end 11.6382 17.568) (width 0.7) (layer "B.Cu") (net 28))
 (segment (start 16.3626 13.9192) (end 16.3626 17.6188) (width 0.7) (layer "B.Cu") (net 28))
 (segment (start 18.6182 13.9192) (end 16.3626 13.9192) (width 0.7) (layer "B.Cu") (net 28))
 (segment (start 16.3626 17.6188) (end 13.975 17.6188) (width 0.7) (layer "B.Cu") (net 28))
 (segment (start 7.2948 16.3742) (end 10.4444 16.3742) (width 0.7) (layer "B.Cu") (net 28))
 (segment (start 11.6382 17.568) (end 13.9242 17.568) (width 0.7) (layer "B.Cu") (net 28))
 (segment (start 13.9242 17.568) (end 13.975 17.6188) (width 0.2) (layer "B.Cu") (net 28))
 (segment (start 3.4632 18.9142) (end 3.3782 18.9992) (width 0.2) (layer "B.Cu") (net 8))
 (segment (start 7.2948 18.9142) (end 3.4632 18.9142) (width 0.7) (layer "B.Cu") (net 8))
 (segment (start 145.1494 58.3438) (end 145.2168 58.4112) (width 0.2) (layer "F.Cu") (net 3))
 (segment (start 21.3664 6.3666) (end 21.3664 18.3262) (width 1.5) (layer "B.Cu") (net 3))
 (segment (start 24.2404 34.633) (end 24.9444 33.929) (width 1) (layer "B.Cu") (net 3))
 (segment (start 24.9444 33.929) (end 32.771 33.929) (width 1.5) (layer "B.Cu") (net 3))
 (segment (start 24.2404 41.7488) (end 24.2404 34.633) (width 1) (layer "B.Cu") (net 3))
 (segment (start 21.3664 18.3262) (end 24.2404 21.2002) (width 1.5) (layer "B.Cu") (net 3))
 (segment (start 24.2404 21.2002) (end 24.2404 41.7488) (width 1.5) (layer "B.Cu") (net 3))
 (segment (start 18.6182 6.2992) (end 21.299 6.2992) (width 1.5) (layer "B.Cu") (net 3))
 (segment (start 12.8524 24.0792) (end 18.6182 24.0792) (width 0.7) (layer "B.Cu") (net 24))
 (segment (start 12.2428 19.1008) (end 12.2428 23.4696) (width 0.7) (layer "B.Cu") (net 24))
 (segment (start 12.2428 23.4696) (end 12.8524 24.0792) (width 0.7) (layer "B.Cu") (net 24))
 (segment (start 13.975 18.8888) (end 12.404 18.8888) (width 0.7) (layer "B.Cu") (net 24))
 (segment (start 12.404 18.8888) (end 12.2174 19.0754) (width 0.5) (layer "B.Cu") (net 24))
 (segment (start 12.2174 19.0754) (end 12.2428 19.1008) (width 0.2) (layer "B.Cu") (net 24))
 (segment (start 137.8254 72.2034) (end 138.0286 72.4066) (width 0.2) (layer "F.Cu") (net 25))
 (segment (start 14.1782 20.362) (end 15.3582 20.362) (width 0.7) (layer "B.Cu") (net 25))
 (segment (start 15.3582 20.362) (end 16.5354 21.5392) (width 0.7) (layer "B.Cu") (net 25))
 (segment (start 16.5354 21.5392) (end 18.6182 21.5392) (width 0.7) (layer "B.Cu") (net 25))
 (segment (start 24.0918 15.663) (end 31.4578 23.029) (width 1.5) (layer "B.Cu") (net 1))
 (segment (start 31.4578 23.029) (end 32.771 23.029) (width 0.2) (layer "B.Cu") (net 1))
 (segment (start 25.4479 6.7535) (end 25.4479 14.3069) (width 1.5) (layer "B.Cu") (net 1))
 (segment (start 25.4479 14.3069) (end 24.0918 15.663) (width 1.5) (layer "B.Cu") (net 1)))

